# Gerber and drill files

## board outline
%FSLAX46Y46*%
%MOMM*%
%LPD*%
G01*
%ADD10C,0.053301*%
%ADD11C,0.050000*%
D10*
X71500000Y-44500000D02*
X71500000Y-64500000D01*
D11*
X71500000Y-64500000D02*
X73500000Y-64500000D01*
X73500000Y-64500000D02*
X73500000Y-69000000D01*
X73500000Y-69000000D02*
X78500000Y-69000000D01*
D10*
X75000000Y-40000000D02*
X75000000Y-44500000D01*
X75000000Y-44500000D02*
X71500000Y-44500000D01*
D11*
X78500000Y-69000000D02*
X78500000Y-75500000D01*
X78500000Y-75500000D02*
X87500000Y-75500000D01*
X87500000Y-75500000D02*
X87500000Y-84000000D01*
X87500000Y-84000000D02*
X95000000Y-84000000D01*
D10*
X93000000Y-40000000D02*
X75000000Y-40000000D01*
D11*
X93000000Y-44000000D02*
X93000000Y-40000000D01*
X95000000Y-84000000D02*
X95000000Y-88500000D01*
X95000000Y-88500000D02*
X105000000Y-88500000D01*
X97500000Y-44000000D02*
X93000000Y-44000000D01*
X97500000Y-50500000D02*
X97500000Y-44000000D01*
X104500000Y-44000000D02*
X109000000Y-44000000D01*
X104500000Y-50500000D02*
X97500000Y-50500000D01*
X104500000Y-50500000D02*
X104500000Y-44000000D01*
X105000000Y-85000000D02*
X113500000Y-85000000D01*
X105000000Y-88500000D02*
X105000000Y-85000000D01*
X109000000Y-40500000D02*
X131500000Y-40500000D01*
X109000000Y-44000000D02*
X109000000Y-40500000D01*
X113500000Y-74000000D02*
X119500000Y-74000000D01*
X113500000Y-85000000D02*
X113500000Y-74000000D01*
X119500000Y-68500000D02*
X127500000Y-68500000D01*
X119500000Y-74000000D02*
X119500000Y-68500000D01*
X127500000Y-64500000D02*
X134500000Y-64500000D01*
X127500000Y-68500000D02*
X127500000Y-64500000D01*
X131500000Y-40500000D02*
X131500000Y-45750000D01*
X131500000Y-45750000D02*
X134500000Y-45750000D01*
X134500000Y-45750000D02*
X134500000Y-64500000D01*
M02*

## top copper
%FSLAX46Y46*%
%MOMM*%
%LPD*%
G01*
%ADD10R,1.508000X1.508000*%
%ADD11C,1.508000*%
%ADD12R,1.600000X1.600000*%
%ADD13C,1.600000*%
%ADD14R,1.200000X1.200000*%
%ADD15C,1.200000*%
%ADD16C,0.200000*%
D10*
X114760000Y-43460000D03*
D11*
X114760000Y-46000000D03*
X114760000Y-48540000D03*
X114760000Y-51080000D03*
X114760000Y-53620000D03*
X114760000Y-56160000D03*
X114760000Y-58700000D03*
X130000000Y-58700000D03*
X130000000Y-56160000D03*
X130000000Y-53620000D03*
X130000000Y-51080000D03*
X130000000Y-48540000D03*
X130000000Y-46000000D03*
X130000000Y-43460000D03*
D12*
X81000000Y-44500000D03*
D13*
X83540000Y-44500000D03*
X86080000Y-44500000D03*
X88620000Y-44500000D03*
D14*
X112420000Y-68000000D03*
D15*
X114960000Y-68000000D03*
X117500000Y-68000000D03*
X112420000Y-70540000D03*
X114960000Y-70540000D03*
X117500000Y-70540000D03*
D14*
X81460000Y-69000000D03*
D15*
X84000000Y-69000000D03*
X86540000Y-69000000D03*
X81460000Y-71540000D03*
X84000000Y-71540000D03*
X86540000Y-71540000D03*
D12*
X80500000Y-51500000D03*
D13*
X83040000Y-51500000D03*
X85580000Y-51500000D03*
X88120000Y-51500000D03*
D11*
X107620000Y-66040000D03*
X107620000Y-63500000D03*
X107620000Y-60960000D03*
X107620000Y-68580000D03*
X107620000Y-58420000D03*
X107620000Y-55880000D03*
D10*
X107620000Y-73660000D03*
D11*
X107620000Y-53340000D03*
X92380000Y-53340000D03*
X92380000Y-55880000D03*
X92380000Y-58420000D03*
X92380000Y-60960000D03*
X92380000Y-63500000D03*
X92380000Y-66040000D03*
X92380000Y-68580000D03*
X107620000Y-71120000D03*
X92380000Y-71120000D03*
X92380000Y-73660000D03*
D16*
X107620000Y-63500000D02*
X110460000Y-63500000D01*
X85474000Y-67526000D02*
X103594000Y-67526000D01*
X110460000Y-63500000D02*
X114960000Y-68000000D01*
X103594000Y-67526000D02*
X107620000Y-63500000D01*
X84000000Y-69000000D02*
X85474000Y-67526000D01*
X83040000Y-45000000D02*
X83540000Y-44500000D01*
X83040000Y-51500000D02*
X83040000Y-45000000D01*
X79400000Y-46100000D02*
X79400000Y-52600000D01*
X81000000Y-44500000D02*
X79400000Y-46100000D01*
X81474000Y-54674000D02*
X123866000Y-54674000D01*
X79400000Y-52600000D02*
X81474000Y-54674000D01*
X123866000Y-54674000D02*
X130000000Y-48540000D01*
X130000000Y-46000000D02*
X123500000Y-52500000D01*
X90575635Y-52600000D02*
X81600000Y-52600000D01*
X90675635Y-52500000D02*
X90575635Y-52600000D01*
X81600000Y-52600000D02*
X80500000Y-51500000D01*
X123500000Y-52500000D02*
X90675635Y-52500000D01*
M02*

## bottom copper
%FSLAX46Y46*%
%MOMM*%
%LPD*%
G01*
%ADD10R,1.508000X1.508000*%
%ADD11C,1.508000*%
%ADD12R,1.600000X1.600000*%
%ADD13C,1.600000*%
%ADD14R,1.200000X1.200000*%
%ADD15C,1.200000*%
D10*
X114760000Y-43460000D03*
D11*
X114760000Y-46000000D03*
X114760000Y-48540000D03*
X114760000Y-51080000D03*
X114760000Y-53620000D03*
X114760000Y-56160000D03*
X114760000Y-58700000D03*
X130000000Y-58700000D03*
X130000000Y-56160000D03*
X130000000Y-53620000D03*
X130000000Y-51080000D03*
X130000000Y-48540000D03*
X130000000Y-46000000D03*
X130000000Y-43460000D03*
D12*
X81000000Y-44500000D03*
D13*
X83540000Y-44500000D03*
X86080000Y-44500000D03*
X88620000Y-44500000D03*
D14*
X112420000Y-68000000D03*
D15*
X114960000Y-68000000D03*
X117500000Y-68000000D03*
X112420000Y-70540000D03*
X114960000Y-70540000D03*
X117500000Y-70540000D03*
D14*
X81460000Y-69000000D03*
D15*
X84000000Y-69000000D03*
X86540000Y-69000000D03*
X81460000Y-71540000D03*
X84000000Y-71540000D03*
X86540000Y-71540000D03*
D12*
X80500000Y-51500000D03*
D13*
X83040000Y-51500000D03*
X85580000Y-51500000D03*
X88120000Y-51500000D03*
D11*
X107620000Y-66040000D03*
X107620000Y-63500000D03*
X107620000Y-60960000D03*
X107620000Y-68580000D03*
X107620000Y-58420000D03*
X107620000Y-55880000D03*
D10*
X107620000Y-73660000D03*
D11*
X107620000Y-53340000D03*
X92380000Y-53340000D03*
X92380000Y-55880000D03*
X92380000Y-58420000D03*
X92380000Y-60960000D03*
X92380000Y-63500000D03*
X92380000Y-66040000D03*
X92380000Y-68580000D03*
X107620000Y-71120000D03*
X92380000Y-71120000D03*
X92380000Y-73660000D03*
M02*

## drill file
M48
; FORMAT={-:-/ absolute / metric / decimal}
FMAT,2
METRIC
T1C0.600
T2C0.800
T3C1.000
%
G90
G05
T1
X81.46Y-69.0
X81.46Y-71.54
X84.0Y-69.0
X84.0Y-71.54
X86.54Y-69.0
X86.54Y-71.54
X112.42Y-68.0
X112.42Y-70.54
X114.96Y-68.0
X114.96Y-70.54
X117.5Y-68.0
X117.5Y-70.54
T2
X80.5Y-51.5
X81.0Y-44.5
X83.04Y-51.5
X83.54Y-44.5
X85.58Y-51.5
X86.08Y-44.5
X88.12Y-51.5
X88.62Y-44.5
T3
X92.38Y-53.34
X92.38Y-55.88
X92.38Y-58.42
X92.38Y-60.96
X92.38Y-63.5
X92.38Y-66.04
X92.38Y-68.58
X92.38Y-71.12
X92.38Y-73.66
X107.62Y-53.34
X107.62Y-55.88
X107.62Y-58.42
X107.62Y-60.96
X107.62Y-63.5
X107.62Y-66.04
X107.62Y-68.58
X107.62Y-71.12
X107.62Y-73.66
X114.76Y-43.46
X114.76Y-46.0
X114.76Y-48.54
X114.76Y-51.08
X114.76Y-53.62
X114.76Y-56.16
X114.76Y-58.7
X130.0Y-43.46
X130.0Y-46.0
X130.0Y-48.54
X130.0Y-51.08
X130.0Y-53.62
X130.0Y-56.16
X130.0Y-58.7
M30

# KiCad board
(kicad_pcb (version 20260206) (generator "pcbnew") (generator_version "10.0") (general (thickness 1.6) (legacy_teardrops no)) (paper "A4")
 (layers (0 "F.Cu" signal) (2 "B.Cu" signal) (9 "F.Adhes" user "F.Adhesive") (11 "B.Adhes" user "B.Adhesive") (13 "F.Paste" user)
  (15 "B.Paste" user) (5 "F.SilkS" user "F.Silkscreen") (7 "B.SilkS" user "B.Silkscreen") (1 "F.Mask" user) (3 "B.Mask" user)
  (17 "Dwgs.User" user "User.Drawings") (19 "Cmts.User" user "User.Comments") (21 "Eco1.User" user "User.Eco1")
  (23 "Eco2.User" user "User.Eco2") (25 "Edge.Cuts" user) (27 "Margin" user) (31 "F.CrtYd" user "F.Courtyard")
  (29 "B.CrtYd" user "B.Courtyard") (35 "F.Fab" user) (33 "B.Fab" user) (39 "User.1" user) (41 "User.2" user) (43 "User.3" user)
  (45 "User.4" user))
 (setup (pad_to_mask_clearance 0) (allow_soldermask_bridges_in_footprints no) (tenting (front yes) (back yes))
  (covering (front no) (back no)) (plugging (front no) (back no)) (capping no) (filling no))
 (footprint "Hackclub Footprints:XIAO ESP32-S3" (layer "F.Cu") (at 122.38 51.0165)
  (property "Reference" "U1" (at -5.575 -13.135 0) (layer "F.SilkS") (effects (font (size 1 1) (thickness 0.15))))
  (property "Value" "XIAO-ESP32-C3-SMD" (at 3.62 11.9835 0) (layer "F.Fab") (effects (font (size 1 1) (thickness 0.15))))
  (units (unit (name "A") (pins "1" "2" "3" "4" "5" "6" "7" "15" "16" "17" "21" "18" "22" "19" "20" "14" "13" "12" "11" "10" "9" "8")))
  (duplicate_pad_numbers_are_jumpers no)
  (pad "1" thru_hole rect (at -7.62 -7.5565) (size 1.508 1.508) (drill 1) (layers "*.Cu" "*.Mask") (remove_unused_layers no)
   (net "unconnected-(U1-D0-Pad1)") (solder_mask_margin 0.102))
  (pad "2" thru_hole circle (at -7.62 -5.0165) (size 1.508 1.508) (drill 1) (layers "*.Cu" "*.Mask") (remove_unused_layers no)
   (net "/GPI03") (solder_mask_margin 0.102))
  (pad "3" thru_hole circle (at -7.62 -2.4765) (size 1.508 1.508) (drill 1) (layers "*.Cu" "*.Mask") (remove_unused_layers no)
   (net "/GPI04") (solder_mask_margin 0.102))
  (pad "4" thru_hole circle (at -7.62 0.0635) (size 1.508 1.508) (drill 1) (layers "*.Cu" "*.Mask") (remove_unused_layers no) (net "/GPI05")
   (solder_mask_margin 0.102))
  (pad "5" thru_hole circle (at -7.62 2.6035) (size 1.508 1.508) (drill 1) (layers "*.Cu" "*.Mask") (remove_unused_layers no) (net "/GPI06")
   (solder_mask_margin 0.102))
  (pad "6" thru_hole circle (at -7.62 5.1435) (size 1.508 1.508) (drill 1) (layers "*.Cu" "*.Mask") (remove_unused_layers no) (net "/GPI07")
   (solder_mask_margin 0.102))
  (pad "7" thru_hole circle (at -7.62 7.6835) (size 1.508 1.508) (drill 1) (layers "*.Cu" "*.Mask") (remove_unused_layers no)
   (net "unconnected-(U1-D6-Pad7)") (solder_mask_margin 0.102))
  (pad "8" thru_hole circle (at 7.62 7.6835) (size 1.508 1.508) (drill 1) (layers "*.Cu" "*.Mask") (remove_unused_layers no)
   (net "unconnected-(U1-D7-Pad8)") (solder_mask_margin 0.102))
  (pad "9" thru_hole circle (at 7.62 5.1435) (size 1.508 1.508) (drill 1) (layers "*.Cu" "*.Mask") (remove_unused_layers no)
   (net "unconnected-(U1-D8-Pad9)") (solder_mask_margin 0.102))
  (pad "10" thru_hole circle (at 7.62 2.6035) (size 1.508 1.508) (drill 1) (layers "*.Cu" "*.Mask") (remove_unused_layers no)
   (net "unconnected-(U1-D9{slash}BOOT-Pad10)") (solder_mask_margin 0.102))
  (pad "11" thru_hole circle (at 7.62 0.0635) (size 1.508 1.508) (drill 1) (layers "*.Cu" "*.Mask") (remove_unused_layers no)
   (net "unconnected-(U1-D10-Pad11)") (solder_mask_margin 0.102))
  (pad "12" thru_hole circle (at 7.62 -2.4765) (size 1.508 1.508) (drill 1) (layers "*.Cu" "*.Mask") (remove_unused_layers no)
   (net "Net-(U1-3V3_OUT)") (solder_mask_margin 0.102))
  (pad "13" thru_hole circle (at 7.62 -5.0165) (size 1.508 1.508) (drill 1) (layers "*.Cu" "*.Mask") (remove_unused_layers no)
   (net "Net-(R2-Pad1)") (solder_mask_margin 0.102))
  (pad "14" thru_hole circle (at 7.62 -7.5565) (size 1.508 1.508) (drill 1) (layers "*.Cu" "*.Mask") (remove_unused_layers no)
   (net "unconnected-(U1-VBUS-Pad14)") (solder_mask_margin 0.102)))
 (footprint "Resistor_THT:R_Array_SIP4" (layer "F.Cu") (at 81 44.5)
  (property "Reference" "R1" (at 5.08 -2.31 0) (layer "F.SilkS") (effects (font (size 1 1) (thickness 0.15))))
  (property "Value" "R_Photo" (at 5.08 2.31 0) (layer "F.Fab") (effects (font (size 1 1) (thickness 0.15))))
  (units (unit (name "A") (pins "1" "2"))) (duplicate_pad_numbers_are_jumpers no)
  (pad "1" thru_hole rect (at 0 0) (size 1.6 1.6) (drill 0.8) (layers "*.Cu" "*.Mask") (remove_unused_layers no) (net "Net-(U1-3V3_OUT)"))
  (pad "2" thru_hole circle (at 2.54 0) (size 1.6 1.6) (drill 0.8) (layers "*.Cu" "*.Mask") (remove_unused_layers no) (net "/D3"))
  (pad "3" thru_hole circle (at 5.08 0) (size 1.6 1.6) (drill 0.8) (layers "*.Cu" "*.Mask") (remove_unused_layers no))
  (pad "4" thru_hole circle (at 7.62 0) (size 1.6 1.6) (drill 0.8) (layers "*.Cu" "*.Mask") (remove_unused_layers no)))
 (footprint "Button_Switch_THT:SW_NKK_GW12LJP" (layer "F.Cu") (at 112.42 68)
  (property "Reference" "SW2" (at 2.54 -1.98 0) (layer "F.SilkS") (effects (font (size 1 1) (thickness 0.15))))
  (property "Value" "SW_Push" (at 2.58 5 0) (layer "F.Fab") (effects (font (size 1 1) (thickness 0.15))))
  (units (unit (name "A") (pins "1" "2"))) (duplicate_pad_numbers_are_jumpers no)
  (pad "1" thru_hole rect (at 0 0) (size 1.2 1.2) (drill 0.6) (layers "*.Cu" "*.Mask") (remove_unused_layers no) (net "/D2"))
  (pad "2" thru_hole circle (at 2.54 0) (size 1.2 1.2) (drill 0.6) (layers "*.Cu" "*.Mask") (remove_unused_layers no) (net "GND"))
  (pad "3" thru_hole circle (at 5.08 0) (size 1.2 1.2) (drill 0.6) (layers "*.Cu" "*.Mask") (remove_unused_layers no))
  (pad "4" thru_hole circle (at 0 2.54) (size 1.2 1.2) (drill 0.6) (layers "*.Cu" "*.Mask") (remove_unused_layers no))
  (pad "5" thru_hole circle (at 2.54 2.54) (size 1.2 1.2) (drill 0.6) (layers "*.Cu" "*.Mask") (remove_unused_layers no))
  (pad "6" thru_hole circle (at 5.08 2.54) (size 1.2 1.2) (drill 0.6) (layers "*.Cu" "*.Mask") (remove_unused_layers no)))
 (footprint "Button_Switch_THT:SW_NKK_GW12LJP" (layer "F.Cu") (at 81.46 69)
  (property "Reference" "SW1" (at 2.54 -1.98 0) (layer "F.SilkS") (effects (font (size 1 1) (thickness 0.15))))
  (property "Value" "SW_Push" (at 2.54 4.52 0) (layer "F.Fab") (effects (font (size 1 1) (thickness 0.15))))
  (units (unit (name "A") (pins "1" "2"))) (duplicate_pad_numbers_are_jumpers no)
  (pad "1" thru_hole rect (at 0 0) (size 1.2 1.2) (drill 0.6) (layers "*.Cu" "*.Mask") (remove_unused_layers no) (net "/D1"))
  (pad "2" thru_hole circle (at 2.54 0) (size 1.2 1.2) (drill 0.6) (layers "*.Cu" "*.Mask") (remove_unused_layers no) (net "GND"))
  (pad "3" thru_hole circle (at 5.08 0) (size 1.2 1.2) (drill 0.6) (layers "*.Cu" "*.Mask") (remove_unused_layers no))
  (pad "4" thru_hole circle (at 0 2.54) (size 1.2 1.2) (drill 0.6) (layers "*.Cu" "*.Mask") (remove_unused_layers no))
  (pad "5" thru_hole circle (at 2.54 2.54) (size 1.2 1.2) (drill 0.6) (layers "*.Cu" "*.Mask") (remove_unused_layers no))
  (pad "6" thru_hole circle (at 5.08 2.54) (size 1.2 1.2) (drill 0.6) (layers "*.Cu" "*.Mask") (remove_unused_layers no)))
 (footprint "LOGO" (layer "F.Cu") (at 79 61)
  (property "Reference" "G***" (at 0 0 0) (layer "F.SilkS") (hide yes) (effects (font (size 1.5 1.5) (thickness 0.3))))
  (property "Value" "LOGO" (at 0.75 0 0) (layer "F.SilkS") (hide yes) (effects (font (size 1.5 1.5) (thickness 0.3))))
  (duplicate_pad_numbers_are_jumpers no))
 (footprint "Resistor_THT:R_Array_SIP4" (layer "F.Cu") (at 80.5 51.5)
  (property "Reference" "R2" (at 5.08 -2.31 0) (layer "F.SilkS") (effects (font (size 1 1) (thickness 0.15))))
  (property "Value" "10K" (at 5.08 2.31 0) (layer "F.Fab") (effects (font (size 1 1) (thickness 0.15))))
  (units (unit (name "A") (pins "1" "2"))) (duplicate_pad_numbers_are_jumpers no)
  (pad "1" thru_hole rect (at 0 0) (size 1.6 1.6) (drill 0.8) (layers "*.Cu" "*.Mask") (remove_unused_layers no) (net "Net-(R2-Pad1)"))
  (pad "2" thru_hole circle (at 2.54 0) (size 1.6 1.6) (drill 0.8) (layers "*.Cu" "*.Mask") (remove_unused_layers no) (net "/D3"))
  (pad "3" thru_hole circle (at 5.08 0) (size 1.6 1.6) (drill 0.8) (layers "*.Cu" "*.Mask") (remove_unused_layers no))
  (pad "4" thru_hole circle (at 7.62 0) (size 1.6 1.6) (drill 0.8) (layers "*.Cu" "*.Mask") (remove_unused_layers no)))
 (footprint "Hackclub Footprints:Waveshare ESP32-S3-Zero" (layer "F.Cu") (at 100 63.5 180)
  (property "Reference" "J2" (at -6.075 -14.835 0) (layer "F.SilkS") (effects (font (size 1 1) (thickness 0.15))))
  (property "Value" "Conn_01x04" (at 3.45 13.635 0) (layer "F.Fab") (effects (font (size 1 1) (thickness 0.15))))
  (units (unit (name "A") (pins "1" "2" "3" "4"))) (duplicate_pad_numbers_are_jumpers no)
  (pad "1" thru_hole circle (at -7.62 -2.54 180) (size 1.508 1.508) (drill 1) (layers "*.Cu" "*.Mask") (remove_unused_layers no)
   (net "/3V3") (solder_mask_margin 0.102))
  (pad "2" thru_hole circle (at -7.62 0 180) (size 1.508 1.508) (drill 1) (layers "*.Cu" "*.Mask") (remove_unused_layers no) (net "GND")
   (solder_mask_margin 0.102))
  (pad "3" thru_hole circle (at -7.62 2.54 180) (size 1.508 1.508) (drill 1) (layers "*.Cu" "*.Mask") (remove_unused_layers no)
   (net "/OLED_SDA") (solder_mask_margin 0.102))
  (pad "3V3" thru_hole circle (at -7.62 -5.08 180) (size 1.508 1.508) (drill 1) (layers "*.Cu" "*.Mask") (remove_unused_layers no)
   (solder_mask_margin 0.102))
  (pad "4" thru_hole circle (at -7.62 5.08 180) (size 1.508 1.508) (drill 1) (layers "*.Cu" "*.Mask") (remove_unused_layers no)
   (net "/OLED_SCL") (solder_mask_margin 0.102))
  (pad "5" thru_hole circle (at -7.62 7.62 180) (size 1.508 1.508) (drill 1) (layers "*.Cu" "*.Mask") (remove_unused_layers no)
   (solder_mask_margin 0.102))
  (pad "5V" thru_hole rect (at -7.62 -10.16 180) (size 1.508 1.508) (drill 1) (layers "*.Cu" "*.Mask") (remove_unused_layers no)
   (solder_mask_margin 0.102))
  (pad "6" thru_hole circle (at -7.62 10.16 180) (size 1.508 1.508) (drill 1) (layers "*.Cu" "*.Mask") (remove_unused_layers no)
   (solder_mask_margin 0.102))
  (pad "7" thru_hole circle (at 7.62 10.16 180) (size 1.508 1.508) (drill 1) (layers "*.Cu" "*.Mask") (remove_unused_layers no)
   (solder_mask_margin 0.102))
  (pad "8" thru_hole circle (at 7.62 7.62 180) (size 1.508 1.508) (drill 1) (layers "*.Cu" "*.Mask") (remove_unused_layers no)
   (solder_mask_margin 0.102))
  (pad "9" thru_hole circle (at 7.62 5.08 180) (size 1.508 1.508) (drill 1) (layers "*.Cu" "*.Mask") (remove_unused_layers no)
   (solder_mask_margin 0.102))
  (pad "10" thru_hole circle (at 7.62 2.54 180) (size 1.508 1.508) (drill 1) (layers "*.Cu" "*.Mask") (remove_unused_layers no)
   (solder_mask_margin 0.102))
  (pad "11" thru_hole circle (at 7.62 0 180) (size 1.508 1.508) (drill 1) (layers "*.Cu" "*.Mask") (remove_unused_layers no)
   (solder_mask_margin 0.102))
  (pad "12" thru_hole circle (at 7.62 -2.54 180) (size 1.508 1.508) (drill 1) (layers "*.Cu" "*.Mask") (remove_unused_layers no)
   (solder_mask_margin 0.102))
  (pad "13" thru_hole circle (at 7.62 -5.08 180) (size 1.508 1.508) (drill 1) (layers "*.Cu" "*.Mask") (remove_unused_layers no)
   (solder_mask_margin 0.102))
  (pad "GND" thru_hole circle (at -7.62 -7.62 180) (size 1.508 1.508) (drill 1) (layers "*.Cu" "*.Mask") (remove_unused_layers no)
   (solder_mask_margin 0.102))
  (pad "RX" thru_hole circle (at 7.62 -7.62 180) (size 1.508 1.508) (drill 1) (layers "*.Cu" "*.Mask") (remove_unused_layers no)
   (solder_mask_margin 0.102))
  (pad "TX" thru_hole circle (at 7.62 -10.16 180) (size 1.508 1.508) (drill 1) (layers "*.Cu" "*.Mask") (remove_unused_layers no)
   (solder_mask_margin 0.102)))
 (gr_line (start 71.5 44.5) (end 71.5 64.5) (stroke (width 0.053301) (type default)) (layer "Edge.Cuts"))
 (gr_line (start 71.5 64.5) (end 73.5 64.5) (stroke (width 0.05) (type default)) (layer "Edge.Cuts"))
 (gr_line (start 73.5 64.5) (end 73.5 69) (stroke (width 0.05) (type default)) (layer "Edge.Cuts"))
 (gr_line (start 73.5 69) (end 78.5 69) (stroke (width 0.05) (type default)) (layer "Edge.Cuts"))
 (gr_line (start 75 40) (end 75 44.5) (stroke (width 0.053301) (type default)) (layer "Edge.Cuts"))
 (gr_line (start 75 44.5) (end 71.5 44.5) (stroke (width 0.053301) (type default)) (layer "Edge.Cuts"))
 (gr_line (start 78.5 69) (end 78.5 75.5) (stroke (width 0.05) (type default)) (layer "Edge.Cuts"))
 (gr_line (start 78.5 75.5) (end 87.5 75.5) (stroke (width 0.05) (type default)) (layer "Edge.Cuts"))
 (gr_line (start 87.5 75.5) (end 87.5 84) (stroke (width 0.05) (type default)) (layer "Edge.Cuts"))
 (gr_line (start 87.5 84) (end 95 84) (stroke (width 0.05) (type default)) (layer "Edge.Cuts"))
 (gr_line (start 93 40) (end 75 40) (stroke (width 0.053301) (type default)) (layer "Edge.Cuts"))
 (gr_line (start 93 44) (end 93 40) (stroke (width 0.05) (type default)) (layer "Edge.Cuts"))
 (gr_line (start 95 84) (end 95 88.5) (stroke (width 0.05) (type default)) (layer "Edge.Cuts"))
 (gr_line (start 95 88.5) (end 105 88.5) (stroke (width 0.05) (type default)) (layer "Edge.Cuts"))
 (gr_line (start 97.5 44) (end 93 44) (stroke (width 0.05) (type default)) (layer "Edge.Cuts"))
 (gr_line (start 97.5 50.5) (end 97.5 44) (stroke (width 0.05) (type default)) (layer "Edge.Cuts"))
 (gr_line (start 104.5 44) (end 109 44) (stroke (width 0.05) (type default)) (layer "Edge.Cuts"))
 (gr_line (start 104.5 50.5) (end 97.5 50.5) (stroke (width 0.05) (type default)) (layer "Edge.Cuts"))
 (gr_line (start 104.5 50.5) (end 104.5 44) (stroke (width 0.05) (type default)) (layer "Edge.Cuts"))
 (gr_line (start 105 85) (end 113.5 85) (stroke (width 0.05) (type default)) (layer "Edge.Cuts"))
 (gr_line (start 105 88.5) (end 105 85) (stroke (width 0.05) (type default)) (layer "Edge.Cuts"))
 (gr_line (start 109 40.5) (end 131.5 40.5) (stroke (width 0.05) (type default)) (layer "Edge.Cuts"))
 (gr_line (start 109 44) (end 109 40.5) (stroke (width 0.05) (type default)) (layer "Edge.Cuts"))
 (gr_line (start 113.5 74) (end 119.5 74) (stroke (width 0.05) (type default)) (layer "Edge.Cuts"))
 (gr_line (start 113.5 85) (end 113.5 74) (stroke (width 0.05) (type default)) (layer "Edge.Cuts"))
 (gr_line (start 119.5 68.5) (end 127.5 68.5) (stroke (width 0.05) (type default)) (layer "Edge.Cuts"))
 (gr_line (start 119.5 74) (end 119.5 68.5) (stroke (width 0.05) (type default)) (layer "Edge.Cuts"))
 (gr_line (start 127.5 64.5) (end 134.5 64.5) (stroke (width 0.05) (type default)) (layer "Edge.Cuts"))
 (gr_line (start 127.5 68.5) (end 127.5 64.5) (stroke (width 0.05) (type default)) (layer "Edge.Cuts"))
 (gr_line (start 131.5 40.5) (end 131.5 45.75) (stroke (width 0.05) (type default)) (layer "Edge.Cuts"))
 (gr_line (start 131.5 45.75) (end 134.5 45.75) (stroke (width 0.05) (type default)) (layer "Edge.Cuts"))
 (gr_line (start 134.5 45.75) (end 134.5 64.5) (stroke (width 0.05) (type default)) (layer "Edge.Cuts"))
 (segment (start 107.62 63.5) (end 110.46 63.5) (width 0.2) (layer "F.Cu") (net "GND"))
 (segment (start 85.474 67.526) (end 103.594 67.526) (width 0.2) (layer "F.Cu") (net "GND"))
 (segment (start 110.46 63.5) (end 114.96 68) (width 0.2) (layer "F.Cu") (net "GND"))
 (segment (start 103.594 67.526) (end 107.62 63.5) (width 0.2) (layer "F.Cu") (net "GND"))
 (segment (start 84 69) (end 85.474 67.526) (width 0.2) (layer "F.Cu") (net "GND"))
 (segment (start 83.04 45) (end 83.54 44.5) (width 0.2) (layer "F.Cu") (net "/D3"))
 (segment (start 83.04 51.5) (end 83.04 45) (width 0.2) (layer "F.Cu") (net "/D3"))
 (segment (start 79.4 46.1) (end 79.4 52.6) (width 0.2) (layer "F.Cu") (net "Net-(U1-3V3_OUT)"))
 (segment (start 81 44.5) (end 79.4 46.1) (width 0.2) (layer "F.Cu") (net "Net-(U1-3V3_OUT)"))
 (segment (start 81.474 54.674) (end 123.866 54.674) (width 0.2) (layer "F.Cu") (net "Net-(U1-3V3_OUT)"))
 (segment (start 79.4 52.6) (end 81.474 54.674) (width 0.2) (layer "F.Cu") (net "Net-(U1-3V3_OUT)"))
 (segment (start 123.866 54.674) (end 130 48.54) (width 0.2) (layer "F.Cu") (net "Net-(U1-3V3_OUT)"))
 (segment (start 130 46) (end 123.5 52.5) (width 0.2) (layer "F.Cu") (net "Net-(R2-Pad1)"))
 (segment (start 90.575635 52.6) (end 81.6 52.6) (width 0.2) (layer "F.Cu") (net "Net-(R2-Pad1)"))
 (segment (start 90.675635 52.5) (end 90.575635 52.6) (width 0.2) (layer "F.Cu") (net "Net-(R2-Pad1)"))
 (segment (start 81.6 52.6) (end 80.5 51.5) (width 0.2) (layer "F.Cu") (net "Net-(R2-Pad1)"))
 (segment (start 123.5 52.5) (end 90.675635 52.5) (width 0.2) (layer "F.Cu") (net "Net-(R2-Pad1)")))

